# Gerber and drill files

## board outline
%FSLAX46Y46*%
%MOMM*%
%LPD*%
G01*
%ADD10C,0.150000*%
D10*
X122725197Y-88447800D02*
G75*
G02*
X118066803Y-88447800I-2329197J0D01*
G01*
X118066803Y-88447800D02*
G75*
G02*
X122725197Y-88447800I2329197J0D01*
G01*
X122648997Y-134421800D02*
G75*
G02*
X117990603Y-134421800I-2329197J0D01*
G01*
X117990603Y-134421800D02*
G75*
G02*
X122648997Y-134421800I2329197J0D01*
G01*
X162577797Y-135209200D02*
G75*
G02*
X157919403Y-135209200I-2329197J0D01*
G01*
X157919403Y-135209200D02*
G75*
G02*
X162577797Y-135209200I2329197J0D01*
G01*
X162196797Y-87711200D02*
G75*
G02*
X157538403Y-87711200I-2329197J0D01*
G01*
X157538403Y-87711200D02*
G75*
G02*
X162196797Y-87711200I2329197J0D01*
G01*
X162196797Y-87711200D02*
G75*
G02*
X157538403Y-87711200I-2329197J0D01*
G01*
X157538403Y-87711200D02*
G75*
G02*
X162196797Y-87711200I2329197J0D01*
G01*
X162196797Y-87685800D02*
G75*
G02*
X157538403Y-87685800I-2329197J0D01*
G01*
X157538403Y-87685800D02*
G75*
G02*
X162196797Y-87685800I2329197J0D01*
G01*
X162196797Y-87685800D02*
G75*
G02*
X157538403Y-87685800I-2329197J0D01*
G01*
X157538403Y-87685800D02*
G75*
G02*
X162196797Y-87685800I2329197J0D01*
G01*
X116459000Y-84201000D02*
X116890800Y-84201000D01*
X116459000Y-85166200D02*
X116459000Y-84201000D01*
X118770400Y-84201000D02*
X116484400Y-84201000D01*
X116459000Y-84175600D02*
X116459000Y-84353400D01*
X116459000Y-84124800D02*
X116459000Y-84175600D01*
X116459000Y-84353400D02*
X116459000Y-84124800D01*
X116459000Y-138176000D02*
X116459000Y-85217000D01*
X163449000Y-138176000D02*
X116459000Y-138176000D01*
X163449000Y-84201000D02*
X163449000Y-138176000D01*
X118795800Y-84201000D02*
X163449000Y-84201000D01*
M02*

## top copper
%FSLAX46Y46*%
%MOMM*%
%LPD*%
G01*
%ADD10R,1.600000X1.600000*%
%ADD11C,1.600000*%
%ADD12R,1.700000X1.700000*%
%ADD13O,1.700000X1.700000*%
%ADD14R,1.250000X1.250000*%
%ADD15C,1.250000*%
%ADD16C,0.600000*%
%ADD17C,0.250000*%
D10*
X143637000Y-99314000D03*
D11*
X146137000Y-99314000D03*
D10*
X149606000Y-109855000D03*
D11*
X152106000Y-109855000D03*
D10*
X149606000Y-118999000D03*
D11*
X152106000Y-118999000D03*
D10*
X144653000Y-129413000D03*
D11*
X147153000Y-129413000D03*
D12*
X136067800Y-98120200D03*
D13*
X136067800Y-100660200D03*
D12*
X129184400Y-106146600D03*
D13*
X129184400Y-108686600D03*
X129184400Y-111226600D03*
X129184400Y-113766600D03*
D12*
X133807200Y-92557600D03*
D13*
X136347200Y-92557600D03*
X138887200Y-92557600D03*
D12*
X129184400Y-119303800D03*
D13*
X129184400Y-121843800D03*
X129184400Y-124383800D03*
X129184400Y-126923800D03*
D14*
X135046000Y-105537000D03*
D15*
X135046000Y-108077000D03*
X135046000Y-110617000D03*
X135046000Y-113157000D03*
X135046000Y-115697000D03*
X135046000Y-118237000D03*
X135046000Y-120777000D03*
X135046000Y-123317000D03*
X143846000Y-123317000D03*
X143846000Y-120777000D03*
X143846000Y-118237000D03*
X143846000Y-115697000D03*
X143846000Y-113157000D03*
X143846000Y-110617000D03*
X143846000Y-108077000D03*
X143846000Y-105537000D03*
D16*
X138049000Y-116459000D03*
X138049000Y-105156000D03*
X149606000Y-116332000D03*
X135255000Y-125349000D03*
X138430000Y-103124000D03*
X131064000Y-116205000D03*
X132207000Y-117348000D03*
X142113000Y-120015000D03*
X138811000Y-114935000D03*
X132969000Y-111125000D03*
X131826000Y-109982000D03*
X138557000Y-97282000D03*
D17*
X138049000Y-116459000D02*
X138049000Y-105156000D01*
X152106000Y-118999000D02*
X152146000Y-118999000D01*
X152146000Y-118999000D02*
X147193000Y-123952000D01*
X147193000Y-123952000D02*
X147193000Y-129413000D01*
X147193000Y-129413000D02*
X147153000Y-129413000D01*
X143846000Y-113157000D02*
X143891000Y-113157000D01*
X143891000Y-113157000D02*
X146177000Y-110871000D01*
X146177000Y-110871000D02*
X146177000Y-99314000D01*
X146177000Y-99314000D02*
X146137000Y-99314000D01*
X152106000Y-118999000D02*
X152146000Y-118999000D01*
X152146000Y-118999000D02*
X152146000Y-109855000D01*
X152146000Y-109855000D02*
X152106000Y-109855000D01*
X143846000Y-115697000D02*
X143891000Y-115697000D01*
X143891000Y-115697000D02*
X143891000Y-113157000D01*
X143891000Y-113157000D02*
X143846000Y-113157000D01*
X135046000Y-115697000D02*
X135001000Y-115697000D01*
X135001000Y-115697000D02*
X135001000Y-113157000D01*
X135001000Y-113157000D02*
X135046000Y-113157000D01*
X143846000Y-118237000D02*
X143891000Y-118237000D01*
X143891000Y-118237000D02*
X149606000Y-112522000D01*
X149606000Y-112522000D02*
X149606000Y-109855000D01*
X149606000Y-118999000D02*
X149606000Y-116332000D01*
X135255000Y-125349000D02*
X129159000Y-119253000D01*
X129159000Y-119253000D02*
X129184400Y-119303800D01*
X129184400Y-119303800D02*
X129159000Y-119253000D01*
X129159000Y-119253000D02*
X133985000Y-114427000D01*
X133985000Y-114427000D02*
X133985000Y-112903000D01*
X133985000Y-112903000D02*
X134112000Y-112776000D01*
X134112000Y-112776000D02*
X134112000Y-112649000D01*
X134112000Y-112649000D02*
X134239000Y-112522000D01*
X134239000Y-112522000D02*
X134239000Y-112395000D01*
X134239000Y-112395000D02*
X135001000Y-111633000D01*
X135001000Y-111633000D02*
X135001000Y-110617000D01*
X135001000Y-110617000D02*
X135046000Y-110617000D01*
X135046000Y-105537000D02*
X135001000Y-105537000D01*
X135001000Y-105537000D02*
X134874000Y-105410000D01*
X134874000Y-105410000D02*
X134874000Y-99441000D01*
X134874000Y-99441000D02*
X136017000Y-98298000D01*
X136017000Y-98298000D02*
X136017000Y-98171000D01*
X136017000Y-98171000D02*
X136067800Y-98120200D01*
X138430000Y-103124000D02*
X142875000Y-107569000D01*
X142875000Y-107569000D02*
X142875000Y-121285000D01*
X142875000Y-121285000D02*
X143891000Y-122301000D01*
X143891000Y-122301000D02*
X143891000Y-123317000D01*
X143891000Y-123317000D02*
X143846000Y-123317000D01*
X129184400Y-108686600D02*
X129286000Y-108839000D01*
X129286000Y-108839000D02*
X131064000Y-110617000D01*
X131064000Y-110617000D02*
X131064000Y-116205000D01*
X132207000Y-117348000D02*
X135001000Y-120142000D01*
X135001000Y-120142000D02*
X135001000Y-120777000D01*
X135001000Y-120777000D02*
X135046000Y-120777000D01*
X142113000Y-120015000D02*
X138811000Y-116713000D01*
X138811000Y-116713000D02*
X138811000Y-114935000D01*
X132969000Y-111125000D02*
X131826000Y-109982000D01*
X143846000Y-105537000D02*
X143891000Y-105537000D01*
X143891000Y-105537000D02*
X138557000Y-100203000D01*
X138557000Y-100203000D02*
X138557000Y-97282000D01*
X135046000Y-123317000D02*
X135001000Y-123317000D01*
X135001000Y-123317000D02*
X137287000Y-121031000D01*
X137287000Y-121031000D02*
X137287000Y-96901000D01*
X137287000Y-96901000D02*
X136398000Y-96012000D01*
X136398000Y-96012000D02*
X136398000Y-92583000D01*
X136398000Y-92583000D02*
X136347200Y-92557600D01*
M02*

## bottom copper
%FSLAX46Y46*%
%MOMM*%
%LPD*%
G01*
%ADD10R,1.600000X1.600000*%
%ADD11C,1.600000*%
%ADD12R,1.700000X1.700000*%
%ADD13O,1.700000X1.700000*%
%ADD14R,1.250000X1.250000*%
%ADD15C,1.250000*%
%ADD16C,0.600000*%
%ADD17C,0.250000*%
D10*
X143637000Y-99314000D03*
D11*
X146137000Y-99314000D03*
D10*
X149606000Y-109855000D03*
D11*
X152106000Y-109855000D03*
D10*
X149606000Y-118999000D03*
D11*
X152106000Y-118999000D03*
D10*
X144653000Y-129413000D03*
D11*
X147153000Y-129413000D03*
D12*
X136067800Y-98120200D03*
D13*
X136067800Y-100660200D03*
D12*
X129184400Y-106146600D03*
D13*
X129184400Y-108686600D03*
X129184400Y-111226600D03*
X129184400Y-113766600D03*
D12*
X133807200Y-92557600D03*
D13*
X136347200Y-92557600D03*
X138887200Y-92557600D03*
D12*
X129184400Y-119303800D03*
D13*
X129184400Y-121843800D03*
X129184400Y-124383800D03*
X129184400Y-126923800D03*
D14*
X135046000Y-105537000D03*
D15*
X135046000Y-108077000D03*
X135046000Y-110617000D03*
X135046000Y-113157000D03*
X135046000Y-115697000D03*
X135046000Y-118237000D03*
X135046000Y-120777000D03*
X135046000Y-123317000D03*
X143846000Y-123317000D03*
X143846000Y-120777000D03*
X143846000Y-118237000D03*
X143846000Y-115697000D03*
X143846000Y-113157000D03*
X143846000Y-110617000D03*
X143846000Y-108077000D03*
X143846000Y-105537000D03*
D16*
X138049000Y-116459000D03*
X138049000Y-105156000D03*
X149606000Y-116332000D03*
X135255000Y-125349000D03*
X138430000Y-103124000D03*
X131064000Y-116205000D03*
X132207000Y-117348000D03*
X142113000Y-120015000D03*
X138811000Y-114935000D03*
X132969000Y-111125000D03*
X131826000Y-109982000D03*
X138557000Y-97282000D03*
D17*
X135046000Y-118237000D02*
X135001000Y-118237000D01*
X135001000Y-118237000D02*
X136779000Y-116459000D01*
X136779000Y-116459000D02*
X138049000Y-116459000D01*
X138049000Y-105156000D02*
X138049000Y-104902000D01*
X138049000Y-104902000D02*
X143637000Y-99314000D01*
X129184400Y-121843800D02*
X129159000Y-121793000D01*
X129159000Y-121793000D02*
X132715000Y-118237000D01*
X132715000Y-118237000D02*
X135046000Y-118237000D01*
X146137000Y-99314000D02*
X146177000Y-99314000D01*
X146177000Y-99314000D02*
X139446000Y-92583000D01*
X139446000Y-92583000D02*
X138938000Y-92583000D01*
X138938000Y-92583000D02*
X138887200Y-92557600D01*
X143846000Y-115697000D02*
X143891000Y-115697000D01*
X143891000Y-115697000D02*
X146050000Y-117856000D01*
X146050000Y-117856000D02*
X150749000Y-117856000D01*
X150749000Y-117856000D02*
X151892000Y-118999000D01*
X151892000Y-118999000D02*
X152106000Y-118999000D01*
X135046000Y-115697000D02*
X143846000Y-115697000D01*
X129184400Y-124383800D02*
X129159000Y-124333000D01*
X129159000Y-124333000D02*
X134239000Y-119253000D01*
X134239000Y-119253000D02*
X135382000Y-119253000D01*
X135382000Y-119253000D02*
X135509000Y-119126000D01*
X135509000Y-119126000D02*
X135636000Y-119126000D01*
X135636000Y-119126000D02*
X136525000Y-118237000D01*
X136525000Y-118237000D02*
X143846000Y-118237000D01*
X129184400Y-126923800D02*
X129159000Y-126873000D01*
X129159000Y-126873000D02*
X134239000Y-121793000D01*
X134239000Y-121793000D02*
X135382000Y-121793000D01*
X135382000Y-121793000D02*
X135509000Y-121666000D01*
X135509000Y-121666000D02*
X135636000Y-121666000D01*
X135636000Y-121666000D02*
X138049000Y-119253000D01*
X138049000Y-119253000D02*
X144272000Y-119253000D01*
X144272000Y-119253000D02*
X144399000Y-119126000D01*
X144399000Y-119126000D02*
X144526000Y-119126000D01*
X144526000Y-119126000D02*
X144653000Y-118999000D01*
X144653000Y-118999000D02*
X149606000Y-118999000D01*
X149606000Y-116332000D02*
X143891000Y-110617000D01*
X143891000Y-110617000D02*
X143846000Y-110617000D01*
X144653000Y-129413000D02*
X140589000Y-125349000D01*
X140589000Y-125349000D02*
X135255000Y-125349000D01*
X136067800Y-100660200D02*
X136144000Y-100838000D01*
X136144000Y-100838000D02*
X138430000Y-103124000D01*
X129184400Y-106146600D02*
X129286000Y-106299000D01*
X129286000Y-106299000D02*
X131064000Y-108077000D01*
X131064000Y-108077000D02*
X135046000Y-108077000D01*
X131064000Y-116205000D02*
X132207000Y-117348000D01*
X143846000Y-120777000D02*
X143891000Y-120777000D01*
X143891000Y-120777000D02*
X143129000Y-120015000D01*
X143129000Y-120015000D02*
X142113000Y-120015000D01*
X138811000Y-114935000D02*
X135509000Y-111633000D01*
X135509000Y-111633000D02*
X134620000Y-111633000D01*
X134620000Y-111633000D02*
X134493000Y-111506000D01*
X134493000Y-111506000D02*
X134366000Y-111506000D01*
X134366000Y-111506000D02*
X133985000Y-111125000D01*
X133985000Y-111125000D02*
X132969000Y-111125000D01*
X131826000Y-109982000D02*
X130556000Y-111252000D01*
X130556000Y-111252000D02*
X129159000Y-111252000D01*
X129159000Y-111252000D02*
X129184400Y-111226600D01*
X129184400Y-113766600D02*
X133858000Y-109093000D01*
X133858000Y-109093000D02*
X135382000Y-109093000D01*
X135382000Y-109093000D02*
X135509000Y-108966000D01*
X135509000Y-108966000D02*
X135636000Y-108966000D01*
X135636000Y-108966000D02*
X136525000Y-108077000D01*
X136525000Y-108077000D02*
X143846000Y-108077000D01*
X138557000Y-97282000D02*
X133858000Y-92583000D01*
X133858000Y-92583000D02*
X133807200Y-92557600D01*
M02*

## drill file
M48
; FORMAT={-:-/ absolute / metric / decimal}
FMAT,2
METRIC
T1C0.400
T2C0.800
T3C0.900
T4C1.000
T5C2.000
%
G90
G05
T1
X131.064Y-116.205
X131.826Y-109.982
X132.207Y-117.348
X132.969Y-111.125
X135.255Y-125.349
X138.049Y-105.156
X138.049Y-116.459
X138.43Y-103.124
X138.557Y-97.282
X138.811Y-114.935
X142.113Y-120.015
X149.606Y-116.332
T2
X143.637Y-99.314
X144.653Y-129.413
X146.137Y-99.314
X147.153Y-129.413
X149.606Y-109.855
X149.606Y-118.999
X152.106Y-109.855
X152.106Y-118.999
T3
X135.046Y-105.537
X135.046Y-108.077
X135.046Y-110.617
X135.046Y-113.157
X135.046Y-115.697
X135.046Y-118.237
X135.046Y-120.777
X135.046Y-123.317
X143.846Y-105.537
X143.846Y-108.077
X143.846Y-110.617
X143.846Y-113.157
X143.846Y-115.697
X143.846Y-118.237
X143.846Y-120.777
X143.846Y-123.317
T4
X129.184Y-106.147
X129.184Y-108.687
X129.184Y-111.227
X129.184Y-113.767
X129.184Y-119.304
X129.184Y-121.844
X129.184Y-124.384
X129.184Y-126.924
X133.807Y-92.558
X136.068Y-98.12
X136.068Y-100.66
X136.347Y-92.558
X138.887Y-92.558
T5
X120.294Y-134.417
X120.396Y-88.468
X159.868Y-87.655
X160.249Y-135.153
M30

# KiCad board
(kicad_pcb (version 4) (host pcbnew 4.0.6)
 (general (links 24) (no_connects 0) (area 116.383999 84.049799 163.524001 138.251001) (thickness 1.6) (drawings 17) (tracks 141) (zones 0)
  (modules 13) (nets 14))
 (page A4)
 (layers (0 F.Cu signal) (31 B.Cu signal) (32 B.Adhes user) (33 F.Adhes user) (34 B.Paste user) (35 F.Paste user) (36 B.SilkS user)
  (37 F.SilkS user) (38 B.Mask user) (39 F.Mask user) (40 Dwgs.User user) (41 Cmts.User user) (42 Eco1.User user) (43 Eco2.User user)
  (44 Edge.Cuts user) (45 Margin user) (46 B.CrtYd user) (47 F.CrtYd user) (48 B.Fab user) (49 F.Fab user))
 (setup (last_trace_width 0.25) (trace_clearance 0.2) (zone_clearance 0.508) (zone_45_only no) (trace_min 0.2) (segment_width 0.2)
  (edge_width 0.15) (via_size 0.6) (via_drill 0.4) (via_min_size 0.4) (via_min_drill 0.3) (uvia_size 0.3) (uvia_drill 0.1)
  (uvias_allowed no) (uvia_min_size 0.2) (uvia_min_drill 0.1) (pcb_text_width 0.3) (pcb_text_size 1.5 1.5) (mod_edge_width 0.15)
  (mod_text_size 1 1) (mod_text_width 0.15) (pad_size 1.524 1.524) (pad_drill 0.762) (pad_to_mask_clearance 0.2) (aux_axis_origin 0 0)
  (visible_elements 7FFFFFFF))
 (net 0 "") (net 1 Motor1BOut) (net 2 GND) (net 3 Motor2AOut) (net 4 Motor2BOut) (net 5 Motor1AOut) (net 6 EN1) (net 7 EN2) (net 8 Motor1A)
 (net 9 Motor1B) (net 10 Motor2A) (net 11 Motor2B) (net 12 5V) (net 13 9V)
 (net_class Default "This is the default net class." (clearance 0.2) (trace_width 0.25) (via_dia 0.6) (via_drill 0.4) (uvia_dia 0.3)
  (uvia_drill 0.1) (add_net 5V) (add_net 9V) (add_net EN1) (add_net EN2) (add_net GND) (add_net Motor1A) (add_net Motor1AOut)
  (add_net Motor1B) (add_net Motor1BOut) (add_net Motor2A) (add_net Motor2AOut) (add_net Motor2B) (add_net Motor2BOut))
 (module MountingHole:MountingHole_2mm (layer F.Cu) (at 159.8676 87.6554)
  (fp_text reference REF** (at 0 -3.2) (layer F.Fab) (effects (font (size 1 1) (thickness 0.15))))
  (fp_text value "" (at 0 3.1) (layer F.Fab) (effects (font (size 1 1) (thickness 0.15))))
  (pad "" np_thru_hole circle (at 0 0) (size 2 2) (drill 2) (layers *.Cu *.Mask)))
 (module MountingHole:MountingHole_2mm (layer F.Cu) (at 120.396 88.4682)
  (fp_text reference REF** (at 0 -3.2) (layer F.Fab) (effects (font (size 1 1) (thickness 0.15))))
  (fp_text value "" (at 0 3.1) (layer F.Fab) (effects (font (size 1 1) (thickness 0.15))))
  (pad "" np_thru_hole circle (at 0 0) (size 2 2) (drill 2) (layers *.Cu *.Mask)))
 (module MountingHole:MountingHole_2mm (layer F.Cu) (at 120.2944 134.4168)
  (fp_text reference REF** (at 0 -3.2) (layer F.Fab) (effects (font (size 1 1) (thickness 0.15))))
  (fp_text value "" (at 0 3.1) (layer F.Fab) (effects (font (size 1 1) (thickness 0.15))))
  (pad "" np_thru_hole circle (at 0 0) (size 2 2) (drill 2) (layers *.Cu *.Mask)))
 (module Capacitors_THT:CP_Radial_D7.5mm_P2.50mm (layer F.Cu) (at 143.637 99.314)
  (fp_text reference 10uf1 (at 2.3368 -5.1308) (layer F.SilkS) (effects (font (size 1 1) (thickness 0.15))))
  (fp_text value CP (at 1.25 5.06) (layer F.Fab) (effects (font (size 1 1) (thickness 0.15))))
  (pad 1 thru_hole rect (at 0 0) (size 1.6 1.6) (drill 0.8) (layers *.Cu *.Mask) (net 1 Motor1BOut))
  (pad 2 thru_hole circle (at 2.5 0) (size 1.6 1.6) (drill 0.8) (layers *.Cu *.Mask) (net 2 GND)))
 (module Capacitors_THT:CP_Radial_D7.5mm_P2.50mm (layer F.Cu) (at 149.606 109.855)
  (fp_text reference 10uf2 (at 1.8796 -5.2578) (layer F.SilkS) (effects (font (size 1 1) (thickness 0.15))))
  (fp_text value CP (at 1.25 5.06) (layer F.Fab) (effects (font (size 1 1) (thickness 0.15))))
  (pad 1 thru_hole rect (at 0 0) (size 1.6 1.6) (drill 0.8) (layers *.Cu *.Mask) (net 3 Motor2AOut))
  (pad 2 thru_hole circle (at 2.5 0) (size 1.6 1.6) (drill 0.8) (layers *.Cu *.Mask) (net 2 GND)))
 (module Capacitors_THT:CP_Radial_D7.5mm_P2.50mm (layer F.Cu) (at 149.606 118.999)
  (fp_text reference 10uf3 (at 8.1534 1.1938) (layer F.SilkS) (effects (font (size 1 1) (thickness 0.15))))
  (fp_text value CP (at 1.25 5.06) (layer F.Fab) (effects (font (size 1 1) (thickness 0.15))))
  (pad 1 thru_hole rect (at 0 0) (size 1.6 1.6) (drill 0.8) (layers *.Cu *.Mask) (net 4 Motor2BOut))
  (pad 2 thru_hole circle (at 2.5 0) (size 1.6 1.6) (drill 0.8) (layers *.Cu *.Mask) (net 2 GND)))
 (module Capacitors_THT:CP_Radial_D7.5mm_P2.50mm (layer F.Cu) (at 144.653 129.413)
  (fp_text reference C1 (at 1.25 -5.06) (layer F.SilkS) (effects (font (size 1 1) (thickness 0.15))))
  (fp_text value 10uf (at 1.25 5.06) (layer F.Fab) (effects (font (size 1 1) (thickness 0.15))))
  (pad 1 thru_hole rect (at 0 0) (size 1.6 1.6) (drill 0.8) (layers *.Cu *.Mask) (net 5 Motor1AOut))
  (pad 2 thru_hole circle (at 2.5 0) (size 1.6 1.6) (drill 0.8) (layers *.Cu *.Mask) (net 2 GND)))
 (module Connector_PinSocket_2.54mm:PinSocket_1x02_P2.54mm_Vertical (layer F.Cu) (at 136.0678 98.1202)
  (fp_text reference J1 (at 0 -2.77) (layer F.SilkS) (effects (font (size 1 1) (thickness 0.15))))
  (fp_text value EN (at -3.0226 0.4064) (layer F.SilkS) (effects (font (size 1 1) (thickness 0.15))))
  (pad 1 thru_hole rect (at 0 0) (size 1.7 1.7) (drill 1) (layers *.Cu *.Mask) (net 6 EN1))
  (pad 2 thru_hole oval (at 0 2.54) (size 1.7 1.7) (drill 1) (layers *.Cu *.Mask) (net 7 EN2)))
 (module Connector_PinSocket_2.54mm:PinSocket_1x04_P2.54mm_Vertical (layer F.Cu) (at 129.1844 106.1466)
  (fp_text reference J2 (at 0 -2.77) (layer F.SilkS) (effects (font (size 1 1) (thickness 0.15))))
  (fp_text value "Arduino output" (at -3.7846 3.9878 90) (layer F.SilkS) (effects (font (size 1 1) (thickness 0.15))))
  (pad 1 thru_hole rect (at 0 0) (size 1.7 1.7) (drill 1) (layers *.Cu *.Mask) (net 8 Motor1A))
  (pad 2 thru_hole oval (at 0 2.54) (size 1.7 1.7) (drill 1) (layers *.Cu *.Mask) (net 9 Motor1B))
  (pad 3 thru_hole oval (at 0 5.08) (size 1.7 1.7) (drill 1) (layers *.Cu *.Mask) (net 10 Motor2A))
  (pad 4 thru_hole oval (at 0 7.62) (size 1.7 1.7) (drill 1) (layers *.Cu *.Mask) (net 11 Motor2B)))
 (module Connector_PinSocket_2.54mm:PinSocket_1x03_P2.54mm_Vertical (layer F.Cu) (at 133.8072 92.5576 90)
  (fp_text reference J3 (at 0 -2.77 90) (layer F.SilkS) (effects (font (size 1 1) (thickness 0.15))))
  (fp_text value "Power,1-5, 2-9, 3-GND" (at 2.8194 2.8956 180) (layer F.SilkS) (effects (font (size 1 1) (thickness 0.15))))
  (pad 1 thru_hole rect (at 0 0 90) (size 1.7 1.7) (drill 1) (layers *.Cu *.Mask) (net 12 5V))
  (pad 2 thru_hole oval (at 0 2.54 90) (size 1.7 1.7) (drill 1) (layers *.Cu *.Mask) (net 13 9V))
  (pad 3 thru_hole oval (at 0 5.08 90) (size 1.7 1.7) (drill 1) (layers *.Cu *.Mask) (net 2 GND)))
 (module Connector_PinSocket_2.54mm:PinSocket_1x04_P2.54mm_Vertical (layer F.Cu) (at 129.1844 119.3038)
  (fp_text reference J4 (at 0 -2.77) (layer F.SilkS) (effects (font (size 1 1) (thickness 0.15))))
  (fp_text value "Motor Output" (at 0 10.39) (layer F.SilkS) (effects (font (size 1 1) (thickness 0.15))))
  (pad 1 thru_hole rect (at 0 0) (size 1.7 1.7) (drill 1) (layers *.Cu *.Mask) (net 5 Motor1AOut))
  (pad 2 thru_hole oval (at 0 2.54) (size 1.7 1.7) (drill 1) (layers *.Cu *.Mask) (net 1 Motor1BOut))
  (pad 3 thru_hole oval (at 0 5.08) (size 1.7 1.7) (drill 1) (layers *.Cu *.Mask) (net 3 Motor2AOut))
  (pad 4 thru_hole oval (at 0 7.62) (size 1.7 1.7) (drill 1) (layers *.Cu *.Mask) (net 4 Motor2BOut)))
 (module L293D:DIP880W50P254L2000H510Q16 (layer F.Cu) (at 139.446 114.427)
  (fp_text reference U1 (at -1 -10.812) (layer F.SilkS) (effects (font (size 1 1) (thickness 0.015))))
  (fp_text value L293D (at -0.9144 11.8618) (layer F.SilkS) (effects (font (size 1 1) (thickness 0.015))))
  (pad 1 thru_hole rect (at -4.4 -8.89) (size 1.25 1.25) (drill 0.9) (layers *.Cu *.Mask) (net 6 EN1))
  (pad 2 thru_hole circle (at -4.4 -6.35) (size 1.25 1.25) (drill 0.9) (layers *.Cu *.Mask) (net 8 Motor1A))
  (pad 3 thru_hole circle (at -4.4 -3.81) (size 1.25 1.25) (drill 0.9) (layers *.Cu *.Mask) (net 5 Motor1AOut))
  (pad 4 thru_hole circle (at -4.4 -1.27) (size 1.25 1.25) (drill 0.9) (layers *.Cu *.Mask) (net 2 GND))
  (pad 5 thru_hole circle (at -4.4 1.27) (size 1.25 1.25) (drill 0.9) (layers *.Cu *.Mask) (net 2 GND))
  (pad 6 thru_hole circle (at -4.4 3.81) (size 1.25 1.25) (drill 0.9) (layers *.Cu *.Mask) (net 1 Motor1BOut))
  (pad 7 thru_hole circle (at -4.4 6.35) (size 1.25 1.25) (drill 0.9) (layers *.Cu *.Mask) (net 9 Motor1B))
  (pad 8 thru_hole circle (at -4.4 8.89) (size 1.25 1.25) (drill 0.9) (layers *.Cu *.Mask) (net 13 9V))
  (pad 9 thru_hole circle (at 4.4 8.89) (size 1.25 1.25) (drill 0.9) (layers *.Cu *.Mask) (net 7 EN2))
  (pad 10 thru_hole circle (at 4.4 6.35) (size 1.25 1.25) (drill 0.9) (layers *.Cu *.Mask) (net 10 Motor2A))
  (pad 11 thru_hole circle (at 4.4 3.81) (size 1.25 1.25) (drill 0.9) (layers *.Cu *.Mask) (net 3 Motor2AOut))
  (pad 12 thru_hole circle (at 4.4 1.27) (size 1.25 1.25) (drill 0.9) (layers *.Cu *.Mask) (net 2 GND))
  (pad 13 thru_hole circle (at 4.4 -1.27) (size 1.25 1.25) (drill 0.9) (layers *.Cu *.Mask) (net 2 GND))
  (pad 14 thru_hole circle (at 4.4 -3.81) (size 1.25 1.25) (drill 0.9) (layers *.Cu *.Mask) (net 4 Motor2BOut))
  (pad 15 thru_hole circle (at 4.4 -6.35) (size 1.25 1.25) (drill 0.9) (layers *.Cu *.Mask) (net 11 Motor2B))
  (pad 16 thru_hole circle (at 4.4 -8.89) (size 1.25 1.25) (drill 0.9) (layers *.Cu *.Mask) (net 12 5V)))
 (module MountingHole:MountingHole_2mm (layer F.Cu) (at 160.2486 135.1534)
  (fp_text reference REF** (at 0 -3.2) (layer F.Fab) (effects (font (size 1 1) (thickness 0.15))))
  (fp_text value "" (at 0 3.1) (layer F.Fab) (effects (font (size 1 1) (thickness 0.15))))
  (pad "" np_thru_hole circle (at 0 0) (size 2 2) (drill 2) (layers *.Cu *.Mask)))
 (gr_circle (center 120.396 88.4478) (end 119.2022 86.4478) (layer Edge.Cuts) (width 0.15))
 (gr_circle (center 120.3198 134.4218) (end 119.126 132.4218) (layer Edge.Cuts) (width 0.15))
 (gr_circle (center 160.2486 135.2092) (end 159.0548 133.2092) (layer Edge.Cuts) (width 0.15))
 (gr_circle (center 159.8676 87.7112) (end 158.6738 85.7112) (layer Edge.Cuts) (width 0.15))
 (gr_circle (center 159.8676 87.7112) (end 158.6738 85.7112) (layer Edge.Cuts) (width 0.15))
 (gr_circle (center 159.8676 87.6858) (end 158.6738 85.6858) (layer Edge.Cuts) (width 0.15))
 (gr_circle (center 159.8676 87.6858) (end 158.6738 85.6858) (layer Edge.Cuts) (width 0.15))
 (gr_line (start 116.459 84.201) (end 116.8908 84.201) (angle 90) (layer Edge.Cuts) (width 0.15))
 (gr_line (start 116.459 85.1662) (end 116.459 84.201) (angle 90) (layer Edge.Cuts) (width 0.15))
 (gr_line (start 118.7704 84.201) (end 116.4844 84.201) (angle 90) (layer Edge.Cuts) (width 0.15))
 (gr_line (start 116.459 84.1756) (end 116.459 84.3534) (angle 90) (layer Edge.Cuts) (width 0.15))
 (gr_line (start 116.459 84.1248) (end 116.459 84.1756) (angle 90) (layer Edge.Cuts) (width 0.15))
 (gr_line (start 116.459 84.3534) (end 116.459 84.1248) (angle 90) (layer Edge.Cuts) (width 0.15))
 (gr_line (start 116.459 138.176) (end 116.459 85.217) (angle 90) (layer Edge.Cuts) (width 0.15))
 (gr_line (start 163.449 138.176) (end 116.459 138.176) (angle 90) (layer Edge.Cuts) (width 0.15))
 (gr_line (start 163.449 84.201) (end 163.449 138.176) (angle 90) (layer Edge.Cuts) (width 0.15))
 (gr_line (start 118.7958 84.201) (end 163.449 84.201) (angle 90) (layer Edge.Cuts) (width 0.15))
 (segment (start 135.046 118.237) (end 135.001 118.237) (width 0.25) (layer B.Cu) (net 1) (status 80000))
 (segment (start 135.001 118.237) (end 136.779 116.459) (width 0.25) (layer B.Cu) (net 1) (status 80000))
 (segment (start 136.779 116.459) (end 138.049 116.459) (width 0.25) (layer B.Cu) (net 1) (status 80000))
 (via (at 138.049 116.459) (size 0.6) (layers F.Cu B.Cu) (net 1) (status 80000))
 (segment (start 138.049 116.459) (end 138.049 105.156) (width 0.25) (layer F.Cu) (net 1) (status 80000))
 (via (at 138.049 105.156) (size 0.6) (layers F.Cu B.Cu) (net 1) (status 80000))
 (segment (start 138.049 105.156) (end 138.049 104.902) (width 0.25) (layer B.Cu) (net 1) (status 80000))
 (segment (start 138.049 104.902) (end 143.637 99.314) (width 0.25) (layer B.Cu) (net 1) (status 80000))
 (segment (start 129.1844 121.8438) (end 129.159 121.793) (width 0.25) (layer B.Cu) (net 1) (status 80000))
 (segment (start 129.159 121.793) (end 132.715 118.237) (width 0.25) (layer B.Cu) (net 1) (status 80000))
 (segment (start 132.715 118.237) (end 135.046 118.237) (width 0.25) (layer B.Cu) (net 1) (status 80000))
 (segment (start 146.137 99.314) (end 146.177 99.314) (width 0.25) (layer B.Cu) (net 2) (status 80000))
 (segment (start 146.177 99.314) (end 139.446 92.583) (width 0.25) (layer B.Cu) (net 2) (status 80000))
 (segment (start 139.446 92.583) (end 138.938 92.583) (width 0.25) (layer B.Cu) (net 2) (status 80000))
 (segment (start 138.938 92.583) (end 138.8872 92.5576) (width 0.25) (layer B.Cu) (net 2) (status 80000))
 (segment (start 152.106 118.999) (end 152.146 118.999) (width 0.25) (layer F.Cu) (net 2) (status 80000))
 (segment (start 152.146 118.999) (end 147.193 123.952) (width 0.25) (layer F.Cu) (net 2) (status 80000))
 (segment (start 147.193 123.952) (end 147.193 129.413) (width 0.25) (layer F.Cu) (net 2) (status 80000))
 (segment (start 147.193 129.413) (end 147.153 129.413) (width 0.25) (layer F.Cu) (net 2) (status 80000))
 (segment (start 143.846 113.157) (end 143.891 113.157) (width 0.25) (layer F.Cu) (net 2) (status 80000))
 (segment (start 143.891 113.157) (end 146.177 110.871) (width 0.25) (layer F.Cu) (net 2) (status 80000))
 (segment (start 146.177 110.871) (end 146.177 99.314) (width 0.25) (layer F.Cu) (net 2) (status 80000))
 (segment (start 146.177 99.314) (end 146.137 99.314) (width 0.25) (layer F.Cu) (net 2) (status 80000))
 (segment (start 143.846 115.697) (end 143.891 115.697) (width 0.25) (layer B.Cu) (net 2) (status 80000))
 (segment (start 143.891 115.697) (end 146.05 117.856) (width 0.25) (layer B.Cu) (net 2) (status 80000))
 (segment (start 146.05 117.856) (end 150.749 117.856) (width 0.25) (layer B.Cu) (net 2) (status 80000))
 (segment (start 150.749 117.856) (end 151.892 118.999) (width 0.25) (layer B.Cu) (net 2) (status 80000))
 (segment (start 151.892 118.999) (end 152.106 118.999) (width 0.25) (layer B.Cu) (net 2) (status 80000))
 (segment (start 152.106 118.999) (end 152.146 118.999) (width 0.25) (layer F.Cu) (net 2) (status 80000))
 (segment (start 152.146 118.999) (end 152.146 109.855) (width 0.25) (layer F.Cu) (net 2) (status 80000))
 (segment (start 152.146 109.855) (end 152.106 109.855) (width 0.25) (layer F.Cu) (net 2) (status 80000))
 (segment (start 135.046 115.697) (end 143.846 115.697) (width 0.25) (layer B.Cu) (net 2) (status 80000))
 (segment (start 143.846 115.697) (end 143.891 115.697) (width 0.25) (layer F.Cu) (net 2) (status 80000))
 (segment (start 143.891 115.697) (end 143.891 113.157) (width 0.25) (layer F.Cu) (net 2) (status 80000))
 (segment (start 143.891 113.157) (end 143.846 113.157) (width 0.25) (layer F.Cu) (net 2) (status 80000))
 (segment (start 135.046 115.697) (end 135.001 115.697) (width 0.25) (layer F.Cu) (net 2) (status 80000))
 (segment (start 135.001 115.697) (end 135.001 113.157) (width 0.25) (layer F.Cu) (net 2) (status 80000))
 (segment (start 135.001 113.157) (end 135.046 113.157) (width 0.25) (layer F.Cu) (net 2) (status 80000))
 (segment (start 129.1844 124.3838) (end 129.159 124.333) (width 0.25) (layer B.Cu) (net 3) (status 80000))
 (segment (start 129.159 124.333) (end 134.239 119.253) (width 0.25) (layer B.Cu) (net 3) (status 80000))
 (segment (start 134.239 119.253) (end 135.382 119.253) (width 0.25) (layer B.Cu) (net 3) (status 80000))
 (segment (start 135.382 119.253) (end 135.509 119.126) (width 0.25) (layer B.Cu) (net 3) (status 80000))
 (segment (start 135.509 119.126) (end 135.636 119.126) (width 0.25) (layer B.Cu) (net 3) (status 80000))
 (segment (start 135.636 119.126) (end 136.525 118.237) (width 0.25) (layer B.Cu) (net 3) (status 80000))
 (segment (start 136.525 118.237) (end 143.846 118.237) (width 0.25) (layer B.Cu) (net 3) (status 80000))
 (segment (start 143.846 118.237) (end 143.891 118.237) (width 0.25) (layer F.Cu) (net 3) (status 80000))
 (segment (start 143.891 118.237) (end 149.606 112.522) (width 0.25) (layer F.Cu) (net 3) (status 80000))
 (segment (start 149.606 112.522) (end 149.606 109.855) (width 0.25) (layer F.Cu) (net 3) (status 80000))
 (segment (start 129.1844 126.9238) (end 129.159 126.873) (width 0.25) (layer B.Cu) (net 4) (status 80000))
 (segment (start 129.159 126.873) (end 134.239 121.793) (width 0.25) (layer B.Cu) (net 4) (status 80000))
 (segment (start 134.239 121.793) (end 135.382 121.793) (width 0.25) (layer B.Cu) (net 4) (status 80000))
 (segment (start 135.382 121.793) (end 135.509 121.666) (width 0.25) (layer B.Cu) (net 4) (status 80000))
 (segment (start 135.509 121.666) (end 135.636 121.666) (width 0.25) (layer B.Cu) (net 4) (status 80000))
 (segment (start 135.636 121.666) (end 138.049 119.253) (width 0.25) (layer B.Cu) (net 4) (status 80000))
 (segment (start 138.049 119.253) (end 144.272 119.253) (width 0.25) (layer B.Cu) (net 4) (status 80000))
 (segment (start 144.272 119.253) (end 144.399 119.126) (width 0.25) (layer B.Cu) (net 4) (status 80000))
 (segment (start 144.399 119.126) (end 144.526 119.126) (width 0.25) (layer B.Cu) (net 4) (status 80000))
 (segment (start 144.526 119.126) (end 144.653 118.999) (width 0.25) (layer B.Cu) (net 4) (status 80000))
 (segment (start 144.653 118.999) (end 149.606 118.999) (width 0.25) (layer B.Cu) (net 4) (status 80000))
 (segment (start 149.606 118.999) (end 149.606 116.332) (width 0.25) (layer F.Cu) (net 4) (status 80000))
 (via (at 149.606 116.332) (size 0.6) (layers F.Cu B.Cu) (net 4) (status 80000))
 (segment (start 149.606 116.332) (end 143.891 110.617) (width 0.25) (layer B.Cu) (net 4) (status 80000))
 (segment (start 143.891 110.617) (end 143.846 110.617) (width 0.25) (layer B.Cu) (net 4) (status 80000))
 (segment (start 144.653 129.413) (end 140.589 125.349) (width 0.25) (layer B.Cu) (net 5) (status 80000))
 (segment (start 140.589 125.349) (end 135.255 125.349) (width 0.25) (layer B.Cu) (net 5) (status 80000))
 (via (at 135.255 125.349) (size 0.6) (layers F.Cu B.Cu) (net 5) (status 80000))
 (segment (start 135.255 125.349) (end 129.159 119.253) (width 0.25) (layer F.Cu) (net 5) (status 80000))
 (segment (start 129.159 119.253) (end 129.1844 119.3038) (width 0.25) (layer F.Cu) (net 5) (status 80000))
 (segment (start 129.1844 119.3038) (end 129.159 119.253) (width 0.25) (layer F.Cu) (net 5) (status 80000))
 (segment (start 129.159 119.253) (end 133.985 114.427) (width 0.25) (layer F.Cu) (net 5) (status 80000))
 (segment (start 133.985 114.427) (end 133.985 112.903) (width 0.25) (layer F.Cu) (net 5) (status 80000))
 (segment (start 133.985 112.903) (end 134.112 112.776) (width 0.25) (layer F.Cu) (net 5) (status 80000))
 (segment (start 134.112 112.776) (end 134.112 112.649) (width 0.25) (layer F.Cu) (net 5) (status 80000))
 (segment (start 134.112 112.649) (end 134.239 112.522) (width 0.25) (layer F.Cu) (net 5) (status 80000))
 (segment (start 134.239 112.522) (end 134.239 112.395) (width 0.25) (layer F.Cu) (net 5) (status 80000))
 (segment (start 134.239 112.395) (end 135.001 111.633) (width 0.25) (layer F.Cu) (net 5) (status 80000))
 (segment (start 135.001 111.633) (end 135.001 110.617) (width 0.25) (layer F.Cu) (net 5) (status 80000))
 (segment (start 135.001 110.617) (end 135.046 110.617) (width 0.25) (layer F.Cu) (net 5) (status 80000))
 (segment (start 135.046 105.537) (end 135.001 105.537) (width 0.25) (layer F.Cu) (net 6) (status 80000))
 (segment (start 135.001 105.537) (end 134.874 105.41) (width 0.25) (layer F.Cu) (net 6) (status 80000))
 (segment (start 134.874 105.41) (end 134.874 99.441) (width 0.25) (layer F.Cu) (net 6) (status 80000))
 (segment (start 134.874 99.441) (end 136.017 98.298) (width 0.25) (layer F.Cu) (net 6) (status 80000))
 (segment (start 136.017 98.298) (end 136.017 98.171) (width 0.25) (layer F.Cu) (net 6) (status 80000))
 (segment (start 136.017 98.171) (end 136.0678 98.1202) (width 0.25) (layer F.Cu) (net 6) (status 80000))
 (segment (start 136.0678 100.6602) (end 136.144 100.838) (width 0.25) (layer B.Cu) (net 7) (status 80000))
 (segment (start 136.144 100.838) (end 138.43 103.124) (width 0.25) (layer B.Cu) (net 7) (status 80000))
 (via (at 138.43 103.124) (size 0.6) (layers F.Cu B.Cu) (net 7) (status 80000))
 (segment (start 138.43 103.124) (end 142.875 107.569) (width 0.25) (layer F.Cu) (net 7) (status 80000))
 (segment (start 142.875 107.569) (end 142.875 121.285) (width 0.25) (layer F.Cu) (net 7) (status 80000))
 (segment (start 142.875 121.285) (end 143.891 122.301) (width 0.25) (layer F.Cu) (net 7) (status 80000))
 (segment (start 143.891 122.301) (end 143.891 123.317) (width 0.25) (layer F.Cu) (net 7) (status 80000))
 (segment (start 143.891 123.317) (end 143.846 123.317) (width 0.25) (layer F.Cu) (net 7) (status 80000))
 (segment (start 129.1844 106.1466) (end 129.286 106.299) (width 0.25) (layer B.Cu) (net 8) (status 80000))
 (segment (start 129.286 106.299) (end 131.064 108.077) (width 0.25) (layer B.Cu) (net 8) (status 80000))
 (segment (start 131.064 108.077) (end 135.046 108.077) (width 0.25) (layer B.Cu) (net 8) (status 80000))
 (segment (start 129.1844 108.6866) (end 129.286 108.839) (width 0.25) (layer F.Cu) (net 9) (status 80000))
 (segment (start 129.286 108.839) (end 131.064 110.617) (width 0.25) (layer F.Cu) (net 9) (status 80000))
 (segment (start 131.064 110.617) (end 131.064 116.205) (width 0.25) (layer F.Cu) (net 9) (status 80000))
 (via (at 131.064 116.205) (size 0.6) (layers F.Cu B.Cu) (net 9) (status 80000))
 (segment (start 131.064 116.205) (end 132.207 117.348) (width 0.25) (layer B.Cu) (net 9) (status 80000))
 (via (at 132.207 117.348) (size 0.6) (layers F.Cu B.Cu) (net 9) (status 80000))
 (segment (start 132.207 117.348) (end 135.001 120.142) (width 0.25) (layer F.Cu) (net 9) (status 80000))
 (segment (start 135.001 120.142) (end 135.001 120.777) (width 0.25) (layer F.Cu) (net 9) (status 80000))
 (segment (start 135.001 120.777) (end 135.046 120.777) (width 0.25) (layer F.Cu) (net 9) (status 80000))
 (segment (start 143.846 120.777) (end 143.891 120.777) (width 0.25) (layer B.Cu) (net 10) (status 80000))
 (segment (start 143.891 120.777) (end 143.129 120.015) (width 0.25) (layer B.Cu) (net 10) (status 80000))
 (segment (start 143.129 120.015) (end 142.113 120.015) (width 0.25) (layer B.Cu) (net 10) (status 80000))
 (via (at 142.113 120.015) (size 0.6) (layers F.Cu B.Cu) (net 10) (status 80000))
 (segment (start 142.113 120.015) (end 138.811 116.713) (width 0.25) (layer F.Cu) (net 10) (status 80000))
 (segment (start 138.811 116.713) (end 138.811 114.935) (width 0.25) (layer F.Cu) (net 10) (status 80000))
 (via (at 138.811 114.935) (size 0.6) (layers F.Cu B.Cu) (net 10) (status 80000))
 (segment (start 138.811 114.935) (end 135.509 111.633) (width 0.25) (layer B.Cu) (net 10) (status 80000))
 (segment (start 135.509 111.633) (end 134.62 111.633) (width 0.25) (layer B.Cu) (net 10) (status 80000))
 (segment (start 134.62 111.633) (end 134.493 111.506) (width 0.25) (layer B.Cu) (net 10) (status 80000))
 (segment (start 134.493 111.506) (end 134.366 111.506) (width 0.25) (layer B.Cu) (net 10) (status 80000))
 (segment (start 134.366 111.506) (end 133.985 111.125) (width 0.25) (layer B.Cu) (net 10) (status 80000))
 (segment (start 133.985 111.125) (end 132.969 111.125) (width 0.25) (layer B.Cu) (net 10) (status 80000))
 (via (at 132.969 111.125) (size 0.6) (layers F.Cu B.Cu) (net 10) (status 80000))
 (segment (start 132.969 111.125) (end 131.826 109.982) (width 0.25) (layer F.Cu) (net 10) (status 80000))
 (via (at 131.826 109.982) (size 0.6) (layers F.Cu B.Cu) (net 10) (status 80000))
 (segment (start 131.826 109.982) (end 130.556 111.252) (width 0.25) (layer B.Cu) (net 10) (status 80000))
 (segment (start 130.556 111.252) (end 129.159 111.252) (width 0.25) (layer B.Cu) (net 10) (status 80000))
 (segment (start 129.159 111.252) (end 129.1844 111.2266) (width 0.25) (layer B.Cu) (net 10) (status 80000))
 (segment (start 129.1844 113.7666) (end 133.858 109.093) (width 0.25) (layer B.Cu) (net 11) (status 80000))
 (segment (start 133.858 109.093) (end 135.382 109.093) (width 0.25) (layer B.Cu) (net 11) (status 80000))
 (segment (start 135.382 109.093) (end 135.509 108.966) (width 0.25) (layer B.Cu) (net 11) (status 80000))
 (segment (start 135.509 108.966) (end 135.636 108.966) (width 0.25) (layer B.Cu) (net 11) (status 80000))
 (segment (start 135.636 108.966) (end 136.525 108.077) (width 0.25) (layer B.Cu) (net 11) (status 80000))
 (segment (start 136.525 108.077) (end 143.846 108.077) (width 0.25) (layer B.Cu) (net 11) (status 80000))
 (segment (start 143.846 105.537) (end 143.891 105.537) (width 0.25) (layer F.Cu) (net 12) (status 80000))
 (segment (start 143.891 105.537) (end 138.557 100.203) (width 0.25) (layer F.Cu) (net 12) (status 80000))
 (segment (start 138.557 100.203) (end 138.557 97.282) (width 0.25) (layer F.Cu) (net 12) (status 80000))
 (via (at 138.557 97.282) (size 0.6) (layers F.Cu B.Cu) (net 12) (status 80000))
 (segment (start 138.557 97.282) (end 133.858 92.583) (width 0.25) (layer B.Cu) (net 12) (status 80000))
 (segment (start 133.858 92.583) (end 133.8072 92.5576) (width 0.25) (layer B.Cu) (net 12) (status 80000))
 (segment (start 135.046 123.317) (end 135.001 123.317) (width 0.25) (layer F.Cu) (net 13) (status 80000))
 (segment (start 135.001 123.317) (end 137.287 121.031) (width 0.25) (layer F.Cu) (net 13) (status 80000))
 (segment (start 137.287 121.031) (end 137.287 96.901) (width 0.25) (layer F.Cu) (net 13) (status 80000))
 (segment (start 137.287 96.901) (end 136.398 96.012) (width 0.25) (layer F.Cu) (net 13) (status 80000))
 (segment (start 136.398 96.012) (end 136.398 92.583) (width 0.25) (layer F.Cu) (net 13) (status 80000))
 (segment (start 136.398 92.583) (end 136.3472 92.5576) (width 0.25) (layer F.Cu) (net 13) (status 80000)))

